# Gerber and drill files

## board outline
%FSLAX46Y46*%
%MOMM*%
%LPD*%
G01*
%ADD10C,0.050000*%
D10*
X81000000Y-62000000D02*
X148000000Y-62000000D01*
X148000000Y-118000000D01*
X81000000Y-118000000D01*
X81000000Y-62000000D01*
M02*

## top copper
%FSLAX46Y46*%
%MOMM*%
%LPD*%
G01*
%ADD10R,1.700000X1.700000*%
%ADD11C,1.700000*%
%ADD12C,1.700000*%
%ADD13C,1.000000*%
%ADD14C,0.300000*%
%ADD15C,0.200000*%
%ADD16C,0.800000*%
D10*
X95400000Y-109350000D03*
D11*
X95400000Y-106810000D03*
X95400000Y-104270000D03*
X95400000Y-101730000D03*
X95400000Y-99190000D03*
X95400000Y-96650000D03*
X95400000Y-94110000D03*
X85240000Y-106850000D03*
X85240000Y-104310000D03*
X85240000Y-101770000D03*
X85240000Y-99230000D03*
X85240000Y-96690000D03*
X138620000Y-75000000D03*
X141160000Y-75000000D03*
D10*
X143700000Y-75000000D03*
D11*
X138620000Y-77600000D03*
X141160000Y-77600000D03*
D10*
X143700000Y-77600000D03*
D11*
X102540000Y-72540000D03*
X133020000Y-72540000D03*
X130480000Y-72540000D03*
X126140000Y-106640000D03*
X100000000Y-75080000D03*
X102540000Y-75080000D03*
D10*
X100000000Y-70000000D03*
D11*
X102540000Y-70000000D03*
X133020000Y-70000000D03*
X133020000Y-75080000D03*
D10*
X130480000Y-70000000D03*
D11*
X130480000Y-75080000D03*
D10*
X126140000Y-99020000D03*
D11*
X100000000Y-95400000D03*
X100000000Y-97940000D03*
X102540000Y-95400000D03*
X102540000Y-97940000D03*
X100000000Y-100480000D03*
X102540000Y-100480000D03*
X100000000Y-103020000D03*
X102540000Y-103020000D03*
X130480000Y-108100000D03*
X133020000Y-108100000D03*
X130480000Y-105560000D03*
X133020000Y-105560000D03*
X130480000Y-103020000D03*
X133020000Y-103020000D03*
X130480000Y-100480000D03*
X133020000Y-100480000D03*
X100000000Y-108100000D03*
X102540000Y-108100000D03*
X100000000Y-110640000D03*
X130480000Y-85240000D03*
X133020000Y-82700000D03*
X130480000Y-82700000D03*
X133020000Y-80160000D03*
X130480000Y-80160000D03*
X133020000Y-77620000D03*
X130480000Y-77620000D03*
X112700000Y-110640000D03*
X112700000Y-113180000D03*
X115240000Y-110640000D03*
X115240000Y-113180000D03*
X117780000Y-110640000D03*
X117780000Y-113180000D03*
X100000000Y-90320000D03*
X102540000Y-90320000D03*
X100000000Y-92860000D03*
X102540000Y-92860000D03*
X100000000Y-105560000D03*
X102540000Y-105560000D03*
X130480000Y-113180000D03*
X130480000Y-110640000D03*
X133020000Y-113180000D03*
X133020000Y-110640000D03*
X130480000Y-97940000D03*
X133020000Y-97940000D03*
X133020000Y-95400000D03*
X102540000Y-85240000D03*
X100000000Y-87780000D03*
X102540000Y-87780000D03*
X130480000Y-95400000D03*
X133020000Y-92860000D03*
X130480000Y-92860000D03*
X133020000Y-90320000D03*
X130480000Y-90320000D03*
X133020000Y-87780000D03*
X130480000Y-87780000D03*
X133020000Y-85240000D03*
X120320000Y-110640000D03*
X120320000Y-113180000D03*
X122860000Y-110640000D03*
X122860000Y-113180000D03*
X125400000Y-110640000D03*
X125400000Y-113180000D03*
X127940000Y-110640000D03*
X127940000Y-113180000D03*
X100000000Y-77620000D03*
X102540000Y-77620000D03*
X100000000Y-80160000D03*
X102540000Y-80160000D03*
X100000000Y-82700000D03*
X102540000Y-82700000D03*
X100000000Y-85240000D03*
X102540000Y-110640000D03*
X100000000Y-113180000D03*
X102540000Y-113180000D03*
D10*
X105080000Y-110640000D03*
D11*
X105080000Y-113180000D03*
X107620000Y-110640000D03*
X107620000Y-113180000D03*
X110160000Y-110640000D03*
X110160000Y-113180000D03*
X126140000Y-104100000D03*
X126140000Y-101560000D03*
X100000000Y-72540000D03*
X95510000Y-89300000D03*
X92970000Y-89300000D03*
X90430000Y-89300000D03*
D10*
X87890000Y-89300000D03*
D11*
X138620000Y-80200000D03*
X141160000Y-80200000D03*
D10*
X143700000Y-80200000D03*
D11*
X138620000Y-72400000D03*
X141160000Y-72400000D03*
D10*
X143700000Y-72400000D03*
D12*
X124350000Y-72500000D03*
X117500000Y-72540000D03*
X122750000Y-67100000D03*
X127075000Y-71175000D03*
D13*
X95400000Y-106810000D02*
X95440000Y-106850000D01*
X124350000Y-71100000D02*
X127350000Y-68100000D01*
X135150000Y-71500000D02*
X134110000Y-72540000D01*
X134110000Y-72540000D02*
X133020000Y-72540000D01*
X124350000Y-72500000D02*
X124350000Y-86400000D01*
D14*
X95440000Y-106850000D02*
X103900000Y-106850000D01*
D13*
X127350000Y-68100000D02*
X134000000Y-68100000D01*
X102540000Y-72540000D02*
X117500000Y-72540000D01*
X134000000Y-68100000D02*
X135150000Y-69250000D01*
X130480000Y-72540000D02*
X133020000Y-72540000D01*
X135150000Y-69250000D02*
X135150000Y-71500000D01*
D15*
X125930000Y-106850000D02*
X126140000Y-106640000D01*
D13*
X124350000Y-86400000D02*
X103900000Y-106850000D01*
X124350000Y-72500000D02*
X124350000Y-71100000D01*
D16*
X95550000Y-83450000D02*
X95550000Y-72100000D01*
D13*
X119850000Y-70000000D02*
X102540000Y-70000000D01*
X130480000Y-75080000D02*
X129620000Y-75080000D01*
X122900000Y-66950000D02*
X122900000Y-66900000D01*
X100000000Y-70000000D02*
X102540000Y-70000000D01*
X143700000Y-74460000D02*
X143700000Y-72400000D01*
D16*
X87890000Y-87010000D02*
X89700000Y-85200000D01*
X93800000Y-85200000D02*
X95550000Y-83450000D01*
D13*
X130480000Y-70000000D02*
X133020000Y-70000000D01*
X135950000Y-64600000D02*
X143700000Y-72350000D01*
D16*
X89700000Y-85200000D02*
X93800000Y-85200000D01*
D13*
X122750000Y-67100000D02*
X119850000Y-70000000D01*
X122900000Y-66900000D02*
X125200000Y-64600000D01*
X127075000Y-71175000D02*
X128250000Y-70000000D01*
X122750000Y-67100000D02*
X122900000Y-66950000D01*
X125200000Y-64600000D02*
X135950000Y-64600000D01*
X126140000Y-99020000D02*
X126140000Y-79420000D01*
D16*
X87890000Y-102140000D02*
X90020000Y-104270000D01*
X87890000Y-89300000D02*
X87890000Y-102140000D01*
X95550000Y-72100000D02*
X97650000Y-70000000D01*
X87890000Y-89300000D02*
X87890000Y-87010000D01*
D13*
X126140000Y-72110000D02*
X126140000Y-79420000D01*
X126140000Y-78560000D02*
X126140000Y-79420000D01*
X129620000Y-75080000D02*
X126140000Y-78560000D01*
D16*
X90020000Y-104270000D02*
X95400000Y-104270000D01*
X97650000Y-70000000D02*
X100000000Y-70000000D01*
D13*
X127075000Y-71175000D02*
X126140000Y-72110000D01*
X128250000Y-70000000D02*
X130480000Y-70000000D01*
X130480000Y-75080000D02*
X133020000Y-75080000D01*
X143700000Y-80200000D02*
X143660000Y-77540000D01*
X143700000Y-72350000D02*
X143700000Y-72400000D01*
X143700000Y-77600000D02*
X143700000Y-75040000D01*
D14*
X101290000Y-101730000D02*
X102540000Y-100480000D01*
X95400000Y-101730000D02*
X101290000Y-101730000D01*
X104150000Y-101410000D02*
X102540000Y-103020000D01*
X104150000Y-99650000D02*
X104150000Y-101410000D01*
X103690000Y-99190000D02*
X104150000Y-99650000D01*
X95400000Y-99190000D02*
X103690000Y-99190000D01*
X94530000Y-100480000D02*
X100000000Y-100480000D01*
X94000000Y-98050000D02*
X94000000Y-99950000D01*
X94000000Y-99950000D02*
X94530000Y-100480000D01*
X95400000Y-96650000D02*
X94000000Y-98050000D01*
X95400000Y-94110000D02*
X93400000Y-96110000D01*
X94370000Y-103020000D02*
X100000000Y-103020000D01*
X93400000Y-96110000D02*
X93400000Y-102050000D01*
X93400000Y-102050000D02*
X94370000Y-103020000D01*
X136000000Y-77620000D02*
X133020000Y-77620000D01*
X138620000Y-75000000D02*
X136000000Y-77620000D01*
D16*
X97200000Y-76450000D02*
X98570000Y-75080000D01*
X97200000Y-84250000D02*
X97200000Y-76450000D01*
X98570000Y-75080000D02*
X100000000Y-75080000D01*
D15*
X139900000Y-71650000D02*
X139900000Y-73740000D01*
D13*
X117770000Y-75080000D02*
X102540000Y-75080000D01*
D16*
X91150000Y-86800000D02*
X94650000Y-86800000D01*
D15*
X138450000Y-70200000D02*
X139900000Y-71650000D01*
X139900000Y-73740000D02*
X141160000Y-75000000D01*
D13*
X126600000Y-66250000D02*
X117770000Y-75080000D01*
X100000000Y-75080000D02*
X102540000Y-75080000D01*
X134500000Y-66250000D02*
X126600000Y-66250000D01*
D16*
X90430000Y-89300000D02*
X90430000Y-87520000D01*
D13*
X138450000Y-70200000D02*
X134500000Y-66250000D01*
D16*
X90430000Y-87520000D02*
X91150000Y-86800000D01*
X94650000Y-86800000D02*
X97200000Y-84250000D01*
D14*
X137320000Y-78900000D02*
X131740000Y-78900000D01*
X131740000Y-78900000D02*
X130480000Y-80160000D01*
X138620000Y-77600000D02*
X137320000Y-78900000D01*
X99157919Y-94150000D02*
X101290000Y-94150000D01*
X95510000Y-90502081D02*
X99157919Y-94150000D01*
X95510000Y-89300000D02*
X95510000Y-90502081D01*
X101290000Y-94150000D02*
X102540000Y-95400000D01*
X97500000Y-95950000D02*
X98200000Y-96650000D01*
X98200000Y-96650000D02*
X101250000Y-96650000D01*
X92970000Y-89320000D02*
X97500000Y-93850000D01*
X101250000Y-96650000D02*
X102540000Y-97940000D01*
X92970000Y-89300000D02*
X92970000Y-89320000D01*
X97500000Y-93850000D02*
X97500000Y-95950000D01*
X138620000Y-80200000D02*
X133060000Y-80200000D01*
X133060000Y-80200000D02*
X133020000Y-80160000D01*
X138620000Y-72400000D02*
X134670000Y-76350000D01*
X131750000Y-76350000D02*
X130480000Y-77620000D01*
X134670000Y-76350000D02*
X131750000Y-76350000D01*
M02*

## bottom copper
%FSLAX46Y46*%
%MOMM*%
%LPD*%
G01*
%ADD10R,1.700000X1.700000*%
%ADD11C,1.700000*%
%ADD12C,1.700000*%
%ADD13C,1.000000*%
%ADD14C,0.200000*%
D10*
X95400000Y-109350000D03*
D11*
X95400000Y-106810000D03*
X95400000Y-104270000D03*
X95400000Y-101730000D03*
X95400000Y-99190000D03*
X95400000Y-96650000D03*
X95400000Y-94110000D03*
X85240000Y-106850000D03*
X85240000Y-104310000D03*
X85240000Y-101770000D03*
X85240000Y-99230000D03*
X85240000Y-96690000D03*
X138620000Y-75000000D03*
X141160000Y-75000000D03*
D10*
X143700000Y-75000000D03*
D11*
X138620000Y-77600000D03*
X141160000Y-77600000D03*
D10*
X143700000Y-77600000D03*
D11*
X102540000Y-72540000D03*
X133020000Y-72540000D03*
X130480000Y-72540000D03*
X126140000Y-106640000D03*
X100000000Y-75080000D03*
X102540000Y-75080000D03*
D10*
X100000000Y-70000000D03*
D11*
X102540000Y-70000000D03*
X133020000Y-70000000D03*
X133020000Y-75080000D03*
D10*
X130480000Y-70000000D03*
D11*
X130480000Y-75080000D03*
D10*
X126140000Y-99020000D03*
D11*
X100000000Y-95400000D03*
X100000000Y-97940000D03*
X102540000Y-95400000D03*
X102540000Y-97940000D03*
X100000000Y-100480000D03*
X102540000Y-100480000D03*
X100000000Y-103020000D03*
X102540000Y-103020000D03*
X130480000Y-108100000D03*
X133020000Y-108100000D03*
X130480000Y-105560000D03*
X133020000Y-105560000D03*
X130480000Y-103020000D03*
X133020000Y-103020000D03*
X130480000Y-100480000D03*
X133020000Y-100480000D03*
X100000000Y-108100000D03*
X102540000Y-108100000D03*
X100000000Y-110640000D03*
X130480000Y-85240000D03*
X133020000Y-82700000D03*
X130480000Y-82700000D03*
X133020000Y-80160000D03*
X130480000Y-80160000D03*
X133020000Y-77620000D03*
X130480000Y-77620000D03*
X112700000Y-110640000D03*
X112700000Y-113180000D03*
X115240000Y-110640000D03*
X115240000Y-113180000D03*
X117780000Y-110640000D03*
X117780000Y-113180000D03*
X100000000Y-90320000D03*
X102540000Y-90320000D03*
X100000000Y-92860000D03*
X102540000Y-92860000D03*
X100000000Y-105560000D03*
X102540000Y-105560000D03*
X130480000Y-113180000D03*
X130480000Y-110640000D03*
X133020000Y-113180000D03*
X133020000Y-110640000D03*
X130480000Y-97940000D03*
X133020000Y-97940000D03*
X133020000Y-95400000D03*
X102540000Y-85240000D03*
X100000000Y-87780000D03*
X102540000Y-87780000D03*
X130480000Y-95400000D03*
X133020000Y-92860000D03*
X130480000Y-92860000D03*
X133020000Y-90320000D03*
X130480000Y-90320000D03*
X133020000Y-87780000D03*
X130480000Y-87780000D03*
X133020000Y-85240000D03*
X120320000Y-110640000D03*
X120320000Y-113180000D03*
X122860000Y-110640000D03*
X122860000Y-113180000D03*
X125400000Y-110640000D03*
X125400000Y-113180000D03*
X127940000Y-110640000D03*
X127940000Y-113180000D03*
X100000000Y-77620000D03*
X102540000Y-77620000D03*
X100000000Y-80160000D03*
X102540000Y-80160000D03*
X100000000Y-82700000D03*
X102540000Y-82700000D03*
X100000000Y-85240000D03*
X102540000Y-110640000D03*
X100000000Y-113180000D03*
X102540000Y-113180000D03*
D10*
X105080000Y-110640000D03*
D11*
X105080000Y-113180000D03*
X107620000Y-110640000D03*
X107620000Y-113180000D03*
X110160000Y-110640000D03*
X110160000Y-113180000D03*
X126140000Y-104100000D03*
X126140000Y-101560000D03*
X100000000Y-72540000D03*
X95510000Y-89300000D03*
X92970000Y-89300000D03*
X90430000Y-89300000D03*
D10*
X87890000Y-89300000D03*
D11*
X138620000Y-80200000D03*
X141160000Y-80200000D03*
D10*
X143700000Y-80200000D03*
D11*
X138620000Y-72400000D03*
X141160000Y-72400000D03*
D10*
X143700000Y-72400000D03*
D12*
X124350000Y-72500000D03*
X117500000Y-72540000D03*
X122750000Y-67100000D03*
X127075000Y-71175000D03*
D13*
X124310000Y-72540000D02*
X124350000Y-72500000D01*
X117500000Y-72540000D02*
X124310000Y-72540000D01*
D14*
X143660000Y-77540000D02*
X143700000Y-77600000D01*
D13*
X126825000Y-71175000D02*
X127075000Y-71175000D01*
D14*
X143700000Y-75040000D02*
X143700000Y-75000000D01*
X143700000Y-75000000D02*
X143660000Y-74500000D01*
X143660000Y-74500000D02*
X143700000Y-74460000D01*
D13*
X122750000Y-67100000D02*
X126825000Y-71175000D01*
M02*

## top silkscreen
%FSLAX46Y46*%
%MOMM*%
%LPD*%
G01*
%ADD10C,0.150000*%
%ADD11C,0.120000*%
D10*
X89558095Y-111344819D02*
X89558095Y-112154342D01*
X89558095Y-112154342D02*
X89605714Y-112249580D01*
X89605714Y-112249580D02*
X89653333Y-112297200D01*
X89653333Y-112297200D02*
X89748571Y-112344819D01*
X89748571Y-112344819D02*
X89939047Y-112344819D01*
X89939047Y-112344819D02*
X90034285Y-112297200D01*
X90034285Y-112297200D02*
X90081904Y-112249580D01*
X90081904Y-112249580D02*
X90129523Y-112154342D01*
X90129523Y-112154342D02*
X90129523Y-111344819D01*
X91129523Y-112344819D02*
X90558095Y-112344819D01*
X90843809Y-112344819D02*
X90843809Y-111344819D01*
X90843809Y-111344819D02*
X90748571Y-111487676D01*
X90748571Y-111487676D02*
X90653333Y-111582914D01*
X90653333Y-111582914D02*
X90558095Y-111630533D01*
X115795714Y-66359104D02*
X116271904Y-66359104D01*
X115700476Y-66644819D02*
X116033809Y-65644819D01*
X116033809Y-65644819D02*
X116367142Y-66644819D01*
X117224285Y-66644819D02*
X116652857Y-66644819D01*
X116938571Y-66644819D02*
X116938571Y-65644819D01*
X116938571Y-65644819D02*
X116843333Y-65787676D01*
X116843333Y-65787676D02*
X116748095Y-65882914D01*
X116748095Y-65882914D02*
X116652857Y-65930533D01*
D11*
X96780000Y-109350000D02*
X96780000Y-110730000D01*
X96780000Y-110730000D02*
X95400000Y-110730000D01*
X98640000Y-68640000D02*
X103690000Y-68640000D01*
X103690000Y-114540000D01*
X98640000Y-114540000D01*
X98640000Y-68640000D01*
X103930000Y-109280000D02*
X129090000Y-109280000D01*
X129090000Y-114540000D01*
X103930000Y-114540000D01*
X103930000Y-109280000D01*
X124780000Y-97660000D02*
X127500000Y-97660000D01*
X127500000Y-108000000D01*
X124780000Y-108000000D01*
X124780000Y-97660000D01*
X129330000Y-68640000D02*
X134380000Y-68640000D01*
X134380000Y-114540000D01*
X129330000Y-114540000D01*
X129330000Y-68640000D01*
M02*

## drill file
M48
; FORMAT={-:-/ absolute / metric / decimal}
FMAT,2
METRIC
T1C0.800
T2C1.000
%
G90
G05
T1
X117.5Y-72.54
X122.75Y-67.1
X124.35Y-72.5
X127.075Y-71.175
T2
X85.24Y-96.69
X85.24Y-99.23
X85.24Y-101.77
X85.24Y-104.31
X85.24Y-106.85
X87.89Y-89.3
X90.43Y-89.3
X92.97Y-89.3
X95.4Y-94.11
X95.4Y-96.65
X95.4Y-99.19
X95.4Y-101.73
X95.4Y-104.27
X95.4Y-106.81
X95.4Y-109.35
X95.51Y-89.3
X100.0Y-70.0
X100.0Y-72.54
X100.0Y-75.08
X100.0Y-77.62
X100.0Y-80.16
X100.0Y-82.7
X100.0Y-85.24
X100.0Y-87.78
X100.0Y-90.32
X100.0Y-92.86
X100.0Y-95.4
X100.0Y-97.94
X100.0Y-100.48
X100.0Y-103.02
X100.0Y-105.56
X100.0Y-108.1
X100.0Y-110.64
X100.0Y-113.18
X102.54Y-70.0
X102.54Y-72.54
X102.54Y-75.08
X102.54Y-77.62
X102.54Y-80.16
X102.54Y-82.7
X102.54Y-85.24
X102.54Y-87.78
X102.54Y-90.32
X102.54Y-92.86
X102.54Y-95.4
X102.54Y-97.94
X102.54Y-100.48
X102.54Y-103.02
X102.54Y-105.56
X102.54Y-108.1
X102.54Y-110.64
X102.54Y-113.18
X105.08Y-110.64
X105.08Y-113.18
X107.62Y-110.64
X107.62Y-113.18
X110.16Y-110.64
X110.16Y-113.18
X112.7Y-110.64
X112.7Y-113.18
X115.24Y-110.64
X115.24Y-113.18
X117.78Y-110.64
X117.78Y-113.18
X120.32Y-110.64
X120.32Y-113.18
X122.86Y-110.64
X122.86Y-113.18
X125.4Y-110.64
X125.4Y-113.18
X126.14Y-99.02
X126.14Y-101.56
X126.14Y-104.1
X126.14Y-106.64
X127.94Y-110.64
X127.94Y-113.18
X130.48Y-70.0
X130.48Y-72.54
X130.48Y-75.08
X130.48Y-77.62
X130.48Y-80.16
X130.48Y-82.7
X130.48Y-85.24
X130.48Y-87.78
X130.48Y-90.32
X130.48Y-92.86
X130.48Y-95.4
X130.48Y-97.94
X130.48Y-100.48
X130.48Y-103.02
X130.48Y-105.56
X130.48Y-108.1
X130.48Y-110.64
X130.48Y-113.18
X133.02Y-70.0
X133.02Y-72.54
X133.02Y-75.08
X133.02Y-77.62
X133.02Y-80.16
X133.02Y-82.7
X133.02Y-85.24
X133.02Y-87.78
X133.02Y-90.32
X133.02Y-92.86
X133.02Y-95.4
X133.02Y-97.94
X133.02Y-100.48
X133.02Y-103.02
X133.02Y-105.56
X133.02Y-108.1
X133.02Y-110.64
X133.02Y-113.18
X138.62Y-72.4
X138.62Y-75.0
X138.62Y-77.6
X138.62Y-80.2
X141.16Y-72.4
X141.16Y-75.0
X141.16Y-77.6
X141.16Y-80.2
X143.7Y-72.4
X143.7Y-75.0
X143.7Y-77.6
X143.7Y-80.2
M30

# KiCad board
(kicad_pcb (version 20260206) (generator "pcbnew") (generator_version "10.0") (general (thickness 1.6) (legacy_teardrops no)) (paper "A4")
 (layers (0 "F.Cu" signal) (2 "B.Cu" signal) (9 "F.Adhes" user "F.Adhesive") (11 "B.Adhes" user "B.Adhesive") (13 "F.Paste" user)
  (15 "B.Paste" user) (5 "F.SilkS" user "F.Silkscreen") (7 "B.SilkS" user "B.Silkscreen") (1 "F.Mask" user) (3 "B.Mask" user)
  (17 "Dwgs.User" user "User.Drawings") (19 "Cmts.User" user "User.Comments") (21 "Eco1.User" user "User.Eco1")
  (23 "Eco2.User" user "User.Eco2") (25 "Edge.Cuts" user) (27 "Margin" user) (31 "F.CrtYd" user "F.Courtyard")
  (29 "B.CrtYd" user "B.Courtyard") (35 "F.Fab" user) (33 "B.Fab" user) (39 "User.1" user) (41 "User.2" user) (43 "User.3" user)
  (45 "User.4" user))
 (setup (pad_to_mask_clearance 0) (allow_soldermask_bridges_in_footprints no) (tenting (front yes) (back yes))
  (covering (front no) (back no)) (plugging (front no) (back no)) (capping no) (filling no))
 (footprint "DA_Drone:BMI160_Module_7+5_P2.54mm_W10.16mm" (layer "F.Cu") (at 95.4 109.35 180)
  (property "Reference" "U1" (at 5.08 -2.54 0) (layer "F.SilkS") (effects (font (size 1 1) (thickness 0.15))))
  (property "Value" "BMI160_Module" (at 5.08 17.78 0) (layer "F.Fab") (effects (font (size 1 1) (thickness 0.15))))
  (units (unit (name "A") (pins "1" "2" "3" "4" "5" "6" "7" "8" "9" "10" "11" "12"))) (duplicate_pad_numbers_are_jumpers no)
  (fp_line (start -1.38 0) (end -1.38 -1.38) (stroke (width 0.12) (type default)) (layer "F.SilkS"))
  (fp_line (start -1.38 -1.38) (end 0 -1.38) (stroke (width 0.12) (type default)) (layer "F.SilkS"))
  (pad "1" thru_hole rect (at 0 0 180) (size 1.7 1.7) (drill 1) (layers "*.Cu" "*.Mask") (remove_unused_layers no)
   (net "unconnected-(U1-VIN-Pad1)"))
  (pad "2" thru_hole circle (at 0 2.54 180) (size 1.7 1.7) (drill 1) (layers "*.Cu" "*.Mask") (remove_unused_layers no) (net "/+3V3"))
  (pad "3" thru_hole circle (at 0 5.08 180) (size 1.7 1.7) (drill 1) (layers "*.Cu" "*.Mask") (remove_unused_layers no) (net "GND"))
  (pad "4" thru_hole circle (at 0 7.62 180) (size 1.7 1.7) (drill 1) (layers "*.Cu" "*.Mask") (remove_unused_layers no) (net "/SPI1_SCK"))
  (pad "5" thru_hole circle (at 0 10.16 180) (size 1.7 1.7) (drill 1) (layers "*.Cu" "*.Mask") (remove_unused_layers no) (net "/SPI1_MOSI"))
  (pad "6" thru_hole circle (at 0 12.7 180) (size 1.7 1.7) (drill 1) (layers "*.Cu" "*.Mask") (remove_unused_layers no) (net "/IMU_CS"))
  (pad "7" thru_hole circle (at 0 15.24 180) (size 1.7 1.7) (drill 1) (layers "*.Cu" "*.Mask") (remove_unused_layers no) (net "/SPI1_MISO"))
  (pad "8" thru_hole circle (at 10.16 2.5 180) (size 1.7 1.7) (drill 1) (layers "*.Cu" "*.Mask") (remove_unused_layers no)
   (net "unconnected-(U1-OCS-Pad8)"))
  (pad "9" thru_hole circle (at 10.16 5.04 180) (size 1.7 1.7) (drill 1) (layers "*.Cu" "*.Mask") (remove_unused_layers no)
   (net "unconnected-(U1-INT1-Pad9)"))
  (pad "10" thru_hole circle (at 10.16 7.58 180) (size 1.7 1.7) (drill 1) (layers "*.Cu" "*.Mask") (remove_unused_layers no)
   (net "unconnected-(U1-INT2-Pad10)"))
  (pad "11" thru_hole circle (at 10.16 10.12 180) (size 1.7 1.7) (drill 1) (layers "*.Cu" "*.Mask") (remove_unused_layers no)
   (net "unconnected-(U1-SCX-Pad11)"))
  (pad "12" thru_hole circle (at 10.16 12.66 180) (size 1.7 1.7) (drill 1) (layers "*.Cu" "*.Mask") (remove_unused_layers no)
   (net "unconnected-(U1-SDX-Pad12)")))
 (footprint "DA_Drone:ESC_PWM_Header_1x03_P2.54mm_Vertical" (layer "F.Cu") (at 143.7 75 -90)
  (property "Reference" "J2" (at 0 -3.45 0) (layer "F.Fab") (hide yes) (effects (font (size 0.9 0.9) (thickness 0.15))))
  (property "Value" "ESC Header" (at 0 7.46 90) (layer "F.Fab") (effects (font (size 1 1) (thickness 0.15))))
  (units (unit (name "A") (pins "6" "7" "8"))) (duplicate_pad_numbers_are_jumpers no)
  (pad "6" thru_hole circle (at 0 5.08 270) (size 1.7 1.7) (drill 1) (layers "*.Cu" "*.Mask") (remove_unused_layers no) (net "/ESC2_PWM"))
  (pad "7" thru_hole circle (at 0 2.54 270) (size 1.7 1.7) (drill 1) (layers "*.Cu" "*.Mask") (remove_unused_layers no) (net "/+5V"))
  (pad "8" thru_hole rect (at 0 0 270) (size 1.7 1.7) (drill 1) (layers "*.Cu" "*.Mask") (remove_unused_layers no) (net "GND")))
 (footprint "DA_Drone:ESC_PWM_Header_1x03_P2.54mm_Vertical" (layer "F.Cu") (at 143.7 77.6 -90)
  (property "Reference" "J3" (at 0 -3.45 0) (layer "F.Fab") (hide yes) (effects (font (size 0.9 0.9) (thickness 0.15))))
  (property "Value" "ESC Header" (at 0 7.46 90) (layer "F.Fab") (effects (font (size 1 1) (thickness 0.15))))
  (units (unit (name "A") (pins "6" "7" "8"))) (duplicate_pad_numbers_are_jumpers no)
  (pad "6" thru_hole circle (at 0 5.08 270) (size 1.7 1.7) (drill 1) (layers "*.Cu" "*.Mask") (remove_unused_layers no) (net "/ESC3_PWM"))
  (pad "7" thru_hole circle (at 0 2.54 270) (size 1.7 1.7) (drill 1) (layers "*.Cu" "*.Mask") (remove_unused_layers no)
   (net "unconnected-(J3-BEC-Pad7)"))
  (pad "8" thru_hole rect (at 0 0 270) (size 1.7 1.7) (drill 1) (layers "*.Cu" "*.Mask") (remove_unused_layers no) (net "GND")))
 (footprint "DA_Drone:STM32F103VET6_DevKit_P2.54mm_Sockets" (layer "F.Cu") (at 100 70)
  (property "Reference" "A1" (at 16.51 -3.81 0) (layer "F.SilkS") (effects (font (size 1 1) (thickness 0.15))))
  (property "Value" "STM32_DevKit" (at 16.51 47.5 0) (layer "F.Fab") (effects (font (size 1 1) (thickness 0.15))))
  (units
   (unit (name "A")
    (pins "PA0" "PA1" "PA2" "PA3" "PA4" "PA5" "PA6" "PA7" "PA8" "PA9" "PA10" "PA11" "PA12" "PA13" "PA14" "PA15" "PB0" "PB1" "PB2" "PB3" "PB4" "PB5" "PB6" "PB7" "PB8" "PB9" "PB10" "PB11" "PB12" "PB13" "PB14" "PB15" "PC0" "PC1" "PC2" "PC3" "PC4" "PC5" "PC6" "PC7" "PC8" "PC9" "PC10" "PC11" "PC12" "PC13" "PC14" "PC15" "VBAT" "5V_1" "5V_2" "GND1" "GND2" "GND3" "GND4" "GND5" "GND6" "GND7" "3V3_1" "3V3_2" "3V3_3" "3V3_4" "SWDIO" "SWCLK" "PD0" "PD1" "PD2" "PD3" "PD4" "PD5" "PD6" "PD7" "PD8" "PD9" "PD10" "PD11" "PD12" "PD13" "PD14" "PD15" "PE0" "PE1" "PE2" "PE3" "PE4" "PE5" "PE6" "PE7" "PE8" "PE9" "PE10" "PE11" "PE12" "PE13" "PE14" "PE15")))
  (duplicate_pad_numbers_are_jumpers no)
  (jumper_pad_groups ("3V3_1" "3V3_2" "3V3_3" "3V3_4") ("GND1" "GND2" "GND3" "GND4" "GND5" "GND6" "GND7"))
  (fp_rect (start -1.36 -1.36) (end 3.69 44.54) (stroke (width 0.12) (type solid)) (fill no) (layer "F.SilkS"))
  (fp_rect (start 3.93 39.28) (end 29.09 44.54) (stroke (width 0.12) (type solid)) (fill no) (layer "F.SilkS"))
  (fp_rect (start 24.78 27.66) (end 27.5 38) (stroke (width 0.12) (type solid)) (fill no) (layer "F.SilkS"))
  (fp_rect (start 29.33 -1.36) (end 34.38 44.54) (stroke (width 0.12) (type solid)) (fill no) (layer "F.SilkS"))
  (pad "3V3_1" thru_hole circle (at 2.54 2.54) (size 1.7 1.7) (drill 1) (layers "*.Cu" "*.Mask") (remove_unused_layers no) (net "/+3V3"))
  (pad "3V3_2" thru_hole circle (at 33.02 2.54) (size 1.7 1.7) (drill 1) (layers "*.Cu" "*.Mask") (remove_unused_layers no) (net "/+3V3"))
  (pad "3V3_3" thru_hole circle (at 30.48 2.54) (size 1.7 1.7) (drill 1) (layers "*.Cu" "*.Mask") (remove_unused_layers no) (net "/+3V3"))
  (pad "3V3_4" thru_hole circle (at 26.14 36.64) (size 1.7 1.7) (drill 1) (layers "*.Cu" "*.Mask") (remove_unused_layers no) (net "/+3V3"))
  (pad "5V_1" thru_hole circle (at 0 5.08) (size 1.7 1.7) (drill 1) (layers "*.Cu" "*.Mask") (remove_unused_layers no) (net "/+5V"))
  (pad "5V_2" thru_hole circle (at 2.54 5.08) (size 1.7 1.7) (drill 1) (layers "*.Cu" "*.Mask") (remove_unused_layers no) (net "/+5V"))
  (pad "GND1" thru_hole rect (at 0 0) (size 1.7 1.7) (drill 1) (layers "*.Cu" "*.Mask") (remove_unused_layers no) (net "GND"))
  (pad "GND2" thru_hole circle (at 2.54 0) (size 1.7 1.7) (drill 1) (layers "*.Cu" "*.Mask") (remove_unused_layers no) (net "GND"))
  (pad "GND3" thru_hole circle (at 33.02 0) (size 1.7 1.7) (drill 1) (layers "*.Cu" "*.Mask") (remove_unused_layers no) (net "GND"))
  (pad "GND4" thru_hole circle (at 33.02 5.08) (size 1.7 1.7) (drill 1) (layers "*.Cu" "*.Mask") (remove_unused_layers no) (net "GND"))
  (pad "GND5" thru_hole rect (at 30.48 0) (size 1.7 1.7) (drill 1) (layers "*.Cu" "*.Mask") (remove_unused_layers no) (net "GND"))
  (pad "GND6" thru_hole circle (at 30.48 5.08) (size 1.7 1.7) (drill 1) (layers "*.Cu" "*.Mask") (remove_unused_layers no) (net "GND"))
  (pad "GND7" thru_hole rect (at 26.14 29.02) (size 1.7 1.7) (drill 1) (layers "*.Cu" "*.Mask") (remove_unused_layers no) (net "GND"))
  (pad "PA0" thru_hole circle (at 0 25.4) (size 1.7 1.7) (drill 1) (layers "*.Cu" "*.Mask") (remove_unused_layers no)
   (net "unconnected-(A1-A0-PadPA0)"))
  (pad "PA1" thru_hole circle (at 0 27.94) (size 1.7 1.7) (drill 1) (layers "*.Cu" "*.Mask") (remove_unused_layers no)
   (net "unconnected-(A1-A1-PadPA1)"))
  (pad "PA2" thru_hole circle (at 2.54 25.4) (size 1.7 1.7) (drill 1) (layers "*.Cu" "*.Mask") (remove_unused_layers no)
   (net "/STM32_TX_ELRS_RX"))
  (pad "PA3" thru_hole circle (at 2.54 27.94) (size 1.7 1.7) (drill 1) (layers "*.Cu" "*.Mask") (remove_unused_layers no)
   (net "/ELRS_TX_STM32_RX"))
  (pad "PA4" thru_hole circle (at 0 30.48) (size 1.7 1.7) (drill 1) (layers "*.Cu" "*.Mask") (remove_unused_layers no) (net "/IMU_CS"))
  (pad "PA5" thru_hole circle (at 2.54 30.48) (size 1.7 1.7) (drill 1) (layers "*.Cu" "*.Mask") (remove_unused_layers no) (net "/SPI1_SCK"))
  (pad "PA6" thru_hole circle (at 0 33.02) (size 1.7 1.7) (drill 1) (layers "*.Cu" "*.Mask") (remove_unused_layers no) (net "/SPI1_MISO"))
  (pad "PA7" thru_hole circle (at 2.54 33.02) (size 1.7 1.7) (drill 1) (layers "*.Cu" "*.Mask") (remove_unused_layers no) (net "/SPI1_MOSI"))
  (pad "PA8" thru_hole circle (at 30.48 38.1) (size 1.7 1.7) (drill 1) (layers "*.Cu" "*.Mask") (remove_unused_layers no)
   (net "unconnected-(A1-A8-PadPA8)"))
  (pad "PA9" thru_hole circle (at 33.02 38.1) (size 1.7 1.7) (drill 1) (layers "*.Cu" "*.Mask") (remove_unused_layers no)
   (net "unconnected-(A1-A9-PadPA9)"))
  (pad "PA10" thru_hole circle (at 30.48 35.56) (size 1.7 1.7) (drill 1) (layers "*.Cu" "*.Mask") (remove_unused_layers no)
   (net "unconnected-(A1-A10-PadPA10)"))
  (pad "PA11" thru_hole circle (at 33.02 35.56) (size 1.7 1.7) (drill 1) (layers "*.Cu" "*.Mask") (remove_unused_layers no)
   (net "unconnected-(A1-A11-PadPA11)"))
  (pad "PA12" thru_hole circle (at 30.48 33.02) (size 1.7 1.7) (drill 1) (layers "*.Cu" "*.Mask") (remove_unused_layers no)
   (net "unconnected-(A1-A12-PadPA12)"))
  (pad "PA13" thru_hole circle (at 33.02 33.02) (size 1.7 1.7) (drill 1) (layers "*.Cu" "*.Mask") (remove_unused_layers no)
   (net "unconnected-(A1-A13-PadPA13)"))
  (pad "PA14" thru_hole circle (at 30.48 30.48) (size 1.7 1.7) (drill 1) (layers "*.Cu" "*.Mask") (remove_unused_layers no)
   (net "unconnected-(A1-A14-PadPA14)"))
  (pad "PA15" thru_hole circle (at 33.02 30.48) (size 1.7 1.7) (drill 1) (layers "*.Cu" "*.Mask") (remove_unused_layers no)
   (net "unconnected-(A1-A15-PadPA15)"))
  (pad "PB0" thru_hole circle (at 0 38.1) (size 1.7 1.7) (drill 1) (layers "*.Cu" "*.Mask") (remove_unused_layers no)
   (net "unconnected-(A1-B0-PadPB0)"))
  (pad "PB1" thru_hole circle (at 2.54 38.1) (size 1.7 1.7) (drill 1) (layers "*.Cu" "*.Mask") (remove_unused_layers no)
   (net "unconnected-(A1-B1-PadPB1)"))
  (pad "PB2" thru_hole circle (at 0 40.64) (size 1.7 1.7) (drill 1) (layers "*.Cu" "*.Mask") (remove_unused_layers no)
   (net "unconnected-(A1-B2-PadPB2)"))
  (pad "PB3" thru_hole circle (at 30.48 15.24) (size 1.7 1.7) (drill 1) (layers "*.Cu" "*.Mask") (remove_unused_layers no)
   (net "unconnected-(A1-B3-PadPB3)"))
  (pad "PB4" thru_hole circle (at 33.02 12.7) (size 1.7 1.7) (drill 1) (layers "*.Cu" "*.Mask") (remove_unused_layers no)
   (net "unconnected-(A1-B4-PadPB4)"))
  (pad "PB5" thru_hole circle (at 30.48 12.7) (size 1.7 1.7) (drill 1) (layers "*.Cu" "*.Mask") (remove_unused_layers no)
   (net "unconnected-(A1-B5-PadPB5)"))
  (pad "PB6" thru_hole circle (at 33.02 10.16) (size 1.7 1.7) (drill 1) (layers "*.Cu" "*.Mask") (remove_unused_layers no) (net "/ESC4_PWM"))
  (pad "PB7" thru_hole circle (at 30.48 10.16) (size 1.7 1.7) (drill 1) (layers "*.Cu" "*.Mask") (remove_unused_layers no) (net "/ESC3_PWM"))
  (pad "PB8" thru_hole circle (at 33.02 7.62) (size 1.7 1.7) (drill 1) (layers "*.Cu" "*.Mask") (remove_unused_layers no) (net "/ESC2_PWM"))
  (pad "PB9" thru_hole circle (at 30.48 7.62) (size 1.7 1.7) (drill 1) (layers "*.Cu" "*.Mask") (remove_unused_layers no) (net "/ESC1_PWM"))
  (pad "PB10" thru_hole circle (at 12.7 40.64) (size 1.7 1.7) (drill 1) (layers "*.Cu" "*.Mask") (remove_unused_layers no)
   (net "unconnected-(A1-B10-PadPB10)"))
  (pad "PB11" thru_hole circle (at 12.7 43.18) (size 1.7 1.7) (drill 1) (layers "*.Cu" "*.Mask") (remove_unused_layers no)
   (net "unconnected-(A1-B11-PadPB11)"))
  (pad "PB12" thru_hole circle (at 15.24 40.64) (size 1.7 1.7) (drill 1) (layers "*.Cu" "*.Mask") (remove_unused_layers no)
   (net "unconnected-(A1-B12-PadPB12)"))
  (pad "PB13" thru_hole circle (at 15.24 43.18) (size 1.7 1.7) (drill 1) (layers "*.Cu" "*.Mask") (remove_unused_layers no)
   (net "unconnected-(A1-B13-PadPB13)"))
  (pad "PB14" thru_hole circle (at 17.78 40.64) (size 1.7 1.7) (drill 1) (layers "*.Cu" "*.Mask") (remove_unused_layers no)
   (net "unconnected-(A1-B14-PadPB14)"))
  (pad "PB15" thru_hole circle (at 17.78 43.18) (size 1.7 1.7) (drill 1) (layers "*.Cu" "*.Mask") (remove_unused_layers no)
   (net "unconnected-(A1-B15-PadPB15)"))
  (pad "PC0" thru_hole circle (at 0 20.32) (size 1.7 1.7) (drill 1) (layers "*.Cu" "*.Mask") (remove_unused_layers no)
   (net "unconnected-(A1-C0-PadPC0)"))
  (pad "PC1" thru_hole circle (at 2.54 20.32) (size 1.7 1.7) (drill 1) (layers "*.Cu" "*.Mask") (remove_unused_layers no)
   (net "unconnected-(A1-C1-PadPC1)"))
  (pad "PC2" thru_hole circle (at 0 22.86) (size 1.7 1.7) (drill 1) (layers "*.Cu" "*.Mask") (remove_unused_layers no)
   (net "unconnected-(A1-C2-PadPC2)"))
  (pad "PC3" thru_hole circle (at 2.54 22.86) (size 1.7 1.7) (drill 1) (layers "*.Cu" "*.Mask") (remove_unused_layers no)
   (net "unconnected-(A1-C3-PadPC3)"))
  (pad "PC4" thru_hole circle (at 0 35.56) (size 1.7 1.7) (drill 1) (layers "*.Cu" "*.Mask") (remove_unused_layers no)
   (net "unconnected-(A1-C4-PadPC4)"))
  (pad "PC5" thru_hole circle (at 2.54 35.56) (size 1.7 1.7) (drill 1) (layers "*.Cu" "*.Mask") (remove_unused_layers no)
   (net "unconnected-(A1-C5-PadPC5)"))
  (pad "PC6" thru_hole circle (at 30.48 43.18) (size 1.7 1.7) (drill 1) (layers "*.Cu" "*.Mask") (remove_unused_layers no)
   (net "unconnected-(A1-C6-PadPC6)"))
  (pad "PC7" thru_hole circle (at 30.48 40.64) (size 1.7 1.7) (drill 1) (layers "*.Cu" "*.Mask") (remove_unused_layers no)
   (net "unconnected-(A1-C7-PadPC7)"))
  (pad "PC8" thru_hole circle (at 33.02 43.18) (size 1.7 1.7) (drill 1) (layers "*.Cu" "*.Mask") (remove_unused_layers no)
   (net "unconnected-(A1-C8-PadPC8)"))
  (pad "PC9" thru_hole circle (at 33.02 40.64) (size 1.7 1.7) (drill 1) (layers "*.Cu" "*.Mask") (remove_unused_layers no)
   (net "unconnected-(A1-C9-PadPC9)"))
  (pad "PC10" thru_hole circle (at 30.48 27.94) (size 1.7 1.7) (drill 1) (layers "*.Cu" "*.Mask") (remove_unused_layers no)
   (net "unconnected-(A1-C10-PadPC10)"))
  (pad "PC11" thru_hole circle (at 33.02 27.94) (size 1.7 1.7) (drill 1) (layers "*.Cu" "*.Mask") (remove_unused_layers no)
   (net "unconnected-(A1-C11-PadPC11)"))
  (pad "PC12" thru_hole circle (at 33.02 25.4) (size 1.7 1.7) (drill 1) (layers "*.Cu" "*.Mask") (remove_unused_layers no)
   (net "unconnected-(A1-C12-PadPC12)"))
  (pad "PC13" thru_hole circle (at 2.54 15.24) (size 1.7 1.7) (drill 1) (layers "*.Cu" "*.Mask") (remove_unused_layers no)
   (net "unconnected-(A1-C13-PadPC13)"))
  (pad "PC14" thru_hole circle (at 0 17.78) (size 1.7 1.7) (drill 1) (layers "*.Cu" "*.Mask") (remove_unused_layers no)
   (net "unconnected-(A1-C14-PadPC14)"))
  (pad "PC15" thru_hole circle (at 2.54 17.78) (size 1.7 1.7) (drill 1) (layers "*.Cu" "*.Mask") (remove_unused_layers no)
   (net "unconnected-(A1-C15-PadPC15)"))
  (pad "PD0" thru_hole circle (at 30.48 25.4) (size 1.7 1.7) (drill 1) (layers "*.Cu" "*.Mask") (remove_unused_layers no)
   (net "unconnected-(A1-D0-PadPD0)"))
  (pad "PD1" thru_hole circle (at 33.02 22.86) (size 1.7 1.7) (drill 1) (layers "*.Cu" "*.Mask") (remove_unused_layers no)
   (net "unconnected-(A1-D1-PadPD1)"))
  (pad "PD2" thru_hole circle (at 30.48 22.86) (size 1.7 1.7) (drill 1) (layers "*.Cu" "*.Mask") (remove_unused_layers no)
   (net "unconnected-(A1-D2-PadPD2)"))
  (pad "PD3" thru_hole circle (at 33.02 20.32) (size 1.7 1.7) (drill 1) (layers "*.Cu" "*.Mask") (remove_unused_layers no)
   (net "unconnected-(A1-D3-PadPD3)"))
  (pad "PD4" thru_hole circle (at 30.48 20.32) (size 1.7 1.7) (drill 1) (layers "*.Cu" "*.Mask") (remove_unused_layers no)
   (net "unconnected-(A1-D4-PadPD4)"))
  (pad "PD5" thru_hole circle (at 33.02 17.78) (size 1.7 1.7) (drill 1) (layers "*.Cu" "*.Mask") (remove_unused_layers no)
   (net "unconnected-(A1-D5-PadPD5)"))
  (pad "PD6" thru_hole circle (at 30.48 17.78) (size 1.7 1.7) (drill 1) (layers "*.Cu" "*.Mask") (remove_unused_layers no)
   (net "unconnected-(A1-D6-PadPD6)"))
  (pad "PD7" thru_hole circle (at 33.02 15.24) (size 1.7 1.7) (drill 1) (layers "*.Cu" "*.Mask") (remove_unused_layers no)
   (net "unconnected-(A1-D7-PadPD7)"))
  (pad "PD8" thru_hole circle (at 20.32 40.64) (size 1.7 1.7) (drill 1) (layers "*.Cu" "*.Mask") (remove_unused_layers no)
   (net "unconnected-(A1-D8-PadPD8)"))
  (pad "PD9" thru_hole circle (at 20.32 43.18) (size 1.7 1.7) (drill 1) (layers "*.Cu" "*.Mask") (remove_unused_layers no)
   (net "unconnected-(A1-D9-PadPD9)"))
  (pad "PD10" thru_hole circle (at 22.86 40.64) (size 1.7 1.7) (drill 1) (layers "*.Cu" "*.Mask") (remove_unused_layers no)
   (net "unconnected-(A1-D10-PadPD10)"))
  (pad "PD11" thru_hole circle (at 22.86 43.18) (size 1.7 1.7) (drill 1) (layers "*.Cu" "*.Mask") (remove_unused_layers no)
   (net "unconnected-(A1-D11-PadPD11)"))
  (pad "PD12" thru_hole circle (at 25.4 40.64) (size 1.7 1.7) (drill 1) (layers "*.Cu" "*.Mask") (remove_unused_layers no)
   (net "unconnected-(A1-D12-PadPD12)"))
  (pad "PD13" thru_hole circle (at 25.4 43.18) (size 1.7 1.7) (drill 1) (layers "*.Cu" "*.Mask") (remove_unused_layers no)
   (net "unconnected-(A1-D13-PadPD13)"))
  (pad "PD14" thru_hole circle (at 27.94 40.64) (size 1.7 1.7) (drill 1) (layers "*.Cu" "*.Mask") (remove_unused_layers no)
   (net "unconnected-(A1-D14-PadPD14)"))
  (pad "PD15" thru_hole circle (at 27.94 43.18) (size 1.7 1.7) (drill 1) (layers "*.Cu" "*.Mask") (remove_unused_layers no)
   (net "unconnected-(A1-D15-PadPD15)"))
  (pad "PE0" thru_hole circle (at 0 7.62) (size 1.7 1.7) (drill 1) (layers "*.Cu" "*.Mask") (remove_unused_layers no)
   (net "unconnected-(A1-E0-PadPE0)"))
  (pad "PE1" thru_hole circle (at 2.54 7.62) (size 1.7 1.7) (drill 1) (layers "*.Cu" "*.Mask") (remove_unused_layers no)
   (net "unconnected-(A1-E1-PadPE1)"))
  (pad "PE2" thru_hole circle (at 0 10.16) (size 1.7 1.7) (drill 1) (layers "*.Cu" "*.Mask") (remove_unused_layers no)
   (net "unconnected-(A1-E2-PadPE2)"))
  (pad "PE3" thru_hole circle (at 2.54 10.16) (size 1.7 1.7) (drill 1) (layers "*.Cu" "*.Mask") (remove_unused_layers no)
   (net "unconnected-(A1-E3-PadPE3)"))
  (pad "PE4" thru_hole circle (at 0 12.7) (size 1.7 1.7) (drill 1) (layers "*.Cu" "*.Mask") (remove_unused_layers no)
   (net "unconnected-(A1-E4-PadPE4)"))
  (pad "PE5" thru_hole circle (at 2.54 12.7) (size 1.7 1.7) (drill 1) (layers "*.Cu" "*.Mask") (remove_unused_layers no)
   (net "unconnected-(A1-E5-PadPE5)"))
  (pad "PE6" thru_hole circle (at 0 15.24) (size 1.7 1.7) (drill 1) (layers "*.Cu" "*.Mask") (remove_unused_layers no)
   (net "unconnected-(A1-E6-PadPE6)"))
  (pad "PE7" thru_hole circle (at 2.54 40.64) (size 1.7 1.7) (drill 1) (layers "*.Cu" "*.Mask") (remove_unused_layers no)
   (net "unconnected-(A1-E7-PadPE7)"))
  (pad "PE8" thru_hole circle (at 0 43.18) (size 1.7 1.7) (drill 1) (layers "*.Cu" "*.Mask") (remove_unused_layers no)
   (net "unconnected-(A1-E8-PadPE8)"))
  (pad "PE9" thru_hole circle (at 2.54 43.18) (size 1.7 1.7) (drill 1) (layers "*.Cu" "*.Mask") (remove_unused_layers no)
   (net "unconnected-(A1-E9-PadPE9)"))
  (pad "PE10" thru_hole rect (at 5.08 40.64) (size 1.7 1.7) (drill 1) (layers "*.Cu" "*.Mask") (remove_unused_layers no)
   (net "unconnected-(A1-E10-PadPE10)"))
  (pad "PE11" thru_hole circle (at 5.08 43.18) (size 1.7 1.7) (drill 1) (layers "*.Cu" "*.Mask") (remove_unused_layers no)
   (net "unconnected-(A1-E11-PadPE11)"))
  (pad "PE12" thru_hole circle (at 7.62 40.64) (size 1.7 1.7) (drill 1) (layers "*.Cu" "*.Mask") (remove_unused_layers no)
   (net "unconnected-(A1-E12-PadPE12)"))
  (pad "PE13" thru_hole circle (at 7.62 43.18) (size 1.7 1.7) (drill 1) (layers "*.Cu" "*.Mask") (remove_unused_layers no)
   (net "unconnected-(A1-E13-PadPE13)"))
  (pad "PE14" thru_hole circle (at 10.16 40.64) (size 1.7 1.7) (drill 1) (layers "*.Cu" "*.Mask") (remove_unused_layers no)
   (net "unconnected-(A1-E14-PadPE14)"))
  (pad "PE15" thru_hole circle (at 10.16 43.18) (size 1.7 1.7) (drill 1) (layers "*.Cu" "*.Mask") (remove_unused_layers no)
   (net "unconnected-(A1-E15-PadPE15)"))
  (pad "SWCLK" thru_hole circle (at 26.14 34.1) (size 1.7 1.7) (drill 1) (layers "*.Cu" "*.Mask") (remove_unused_layers no)
   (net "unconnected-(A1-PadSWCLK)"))
  (pad "SWDIO" thru_hole circle (at 26.14 31.56) (size 1.7 1.7) (drill 1) (layers "*.Cu" "*.Mask") (remove_unused_layers no)
   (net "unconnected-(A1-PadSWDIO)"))
  (pad "VBAT" thru_hole circle (at 0 2.54) (size 1.7 1.7) (drill 1) (layers "*.Cu" "*.Mask") (remove_unused_layers no)
   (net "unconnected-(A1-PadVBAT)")))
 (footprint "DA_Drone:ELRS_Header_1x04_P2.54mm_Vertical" (layer "F.Cu") (at 87.89 89.3 90)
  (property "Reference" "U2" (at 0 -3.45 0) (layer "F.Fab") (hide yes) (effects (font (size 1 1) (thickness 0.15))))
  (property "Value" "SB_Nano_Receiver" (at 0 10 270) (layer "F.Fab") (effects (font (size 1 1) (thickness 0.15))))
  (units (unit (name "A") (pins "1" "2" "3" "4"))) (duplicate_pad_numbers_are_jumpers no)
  (pad "1" thru_hole circle (at 0 7.62 90) (size 1.7 1.7) (drill 1) (layers "*.Cu" "*.Mask") (remove_unused_layers no)
   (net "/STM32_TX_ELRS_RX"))
  (pad "2" thru_hole circle (at 0 5.08 90) (size 1.7 1.7) (drill 1) (layers "*.Cu" "*.Mask") (remove_unused_layers no)
   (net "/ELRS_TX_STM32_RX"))
  (pad "3" thru_hole circle (at 0 2.54 90) (size 1.7 1.7) (drill 1) (layers "*.Cu" "*.Mask") (remove_unused_layers no) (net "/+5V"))
  (pad "4" thru_hole rect (at 0 0 90) (size 1.7 1.7) (drill 1) (layers "*.Cu" "*.Mask") (remove_unused_layers no) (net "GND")))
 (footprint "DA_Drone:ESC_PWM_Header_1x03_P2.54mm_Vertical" (layer "F.Cu") (at 143.7 80.2 -90)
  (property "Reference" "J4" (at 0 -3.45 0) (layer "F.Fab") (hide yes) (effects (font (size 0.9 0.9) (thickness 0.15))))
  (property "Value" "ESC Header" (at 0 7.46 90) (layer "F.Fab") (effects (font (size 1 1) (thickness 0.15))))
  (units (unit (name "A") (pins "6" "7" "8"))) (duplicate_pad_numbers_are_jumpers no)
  (pad "6" thru_hole circle (at 0 5.08 270) (size 1.7 1.7) (drill 1) (layers "*.Cu" "*.Mask") (remove_unused_layers no) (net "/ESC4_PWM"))
  (pad "7" thru_hole circle (at 0 2.54 270) (size 1.7 1.7) (drill 1) (layers "*.Cu" "*.Mask") (remove_unused_layers no)
   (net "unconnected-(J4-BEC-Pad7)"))
  (pad "8" thru_hole rect (at 0 0 270) (size 1.7 1.7) (drill 1) (layers "*.Cu" "*.Mask") (remove_unused_layers no) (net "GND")))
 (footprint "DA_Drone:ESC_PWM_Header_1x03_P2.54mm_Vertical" (layer "F.Cu") (at 143.7 72.4 -90)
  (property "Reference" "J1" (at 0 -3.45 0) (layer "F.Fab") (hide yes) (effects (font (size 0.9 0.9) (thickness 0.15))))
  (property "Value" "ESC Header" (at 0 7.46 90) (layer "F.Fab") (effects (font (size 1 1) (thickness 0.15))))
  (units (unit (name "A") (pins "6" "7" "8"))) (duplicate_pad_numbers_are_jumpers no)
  (pad "6" thru_hole circle (at 0 5.08 270) (size 1.7 1.7) (drill 1) (layers "*.Cu" "*.Mask") (remove_unused_layers no) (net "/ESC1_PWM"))
  (pad "7" thru_hole circle (at 0 2.54 270) (size 1.7 1.7) (drill 1) (layers "*.Cu" "*.Mask") (remove_unused_layers no)
   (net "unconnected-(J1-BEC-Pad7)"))
  (pad "8" thru_hole rect (at 0 0 270) (size 1.7 1.7) (drill 1) (layers "*.Cu" "*.Mask") (remove_unused_layers no) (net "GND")))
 (gr_rect (start 81 62) (end 148 118) (stroke (width 0.05) (type default)) (fill no) (layer "Edge.Cuts"))
 (segment (start 95.4 106.81) (end 95.44 106.85) (width 1) (layer "F.Cu") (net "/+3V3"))
 (segment (start 124.35 71.1) (end 127.35 68.1) (width 1) (layer "F.Cu") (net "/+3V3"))
 (segment (start 135.15 71.5) (end 134.11 72.54) (width 1) (layer "F.Cu") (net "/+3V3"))
 (segment (start 134.11 72.54) (end 133.02 72.54) (width 1) (layer "F.Cu") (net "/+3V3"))
 (segment (start 124.35 72.5) (end 124.35 86.4) (width 1) (layer "F.Cu") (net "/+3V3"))
 (segment (start 95.44 106.85) (end 103.9 106.85) (width 0.3) (layer "F.Cu") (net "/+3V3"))
 (segment (start 127.35 68.1) (end 134 68.1) (width 1) (layer "F.Cu") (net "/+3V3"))
 (segment (start 102.54 72.54) (end 117.5 72.54) (width 1) (layer "F.Cu") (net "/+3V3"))
 (segment (start 134 68.1) (end 135.15 69.25) (width 1) (layer "F.Cu") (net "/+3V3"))
 (segment (start 130.48 72.54) (end 133.02 72.54) (width 1) (layer "F.Cu") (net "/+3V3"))
 (segment (start 135.15 69.25) (end 135.15 71.5) (width 1) (layer "F.Cu") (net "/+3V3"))
 (segment (start 125.93 106.85) (end 126.14 106.64) (width 0.2) (layer "F.Cu") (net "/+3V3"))
 (segment (start 124.35 86.4) (end 103.9 106.85) (width 1) (layer "F.Cu") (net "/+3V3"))
 (segment (start 124.35 72.5) (end 124.35 71.1) (width 1) (layer "F.Cu") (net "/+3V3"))
 (via (at 124.35 72.5) (size 1.7) (drill 0.8) (layers "F.Cu" "B.Cu") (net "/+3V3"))
 (via (at 117.5 72.54) (size 1.7) (drill 0.8) (layers "F.Cu" "B.Cu") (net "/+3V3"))
 (segment (start 124.31 72.54) (end 124.35 72.5) (width 1) (layer "B.Cu") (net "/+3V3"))
 (segment (start 117.5 72.54) (end 124.31 72.54) (width 1) (layer "B.Cu") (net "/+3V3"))
 (segment (start 95.55 83.45) (end 95.55 72.1) (width 0.8) (layer "F.Cu") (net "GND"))
 (segment (start 119.85 70) (end 102.54 70) (width 1) (layer "F.Cu") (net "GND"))
 (segment (start 130.48 75.08) (end 129.62 75.08) (width 1) (layer "F.Cu") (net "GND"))
 (segment (start 122.9 66.95) (end 122.9 66.9) (width 1) (layer "F.Cu") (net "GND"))
 (segment (start 100 70) (end 102.54 70) (width 1) (layer "F.Cu") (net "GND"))
 (segment (start 143.7 74.46) (end 143.7 72.4) (width 1) (layer "F.Cu") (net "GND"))
 (segment (start 87.89 87.01) (end 89.7 85.2) (width 0.8) (layer "F.Cu") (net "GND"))
 (segment (start 93.8 85.2) (end 95.55 83.45) (width 0.8) (layer "F.Cu") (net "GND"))
 (segment (start 130.48 70) (end 133.02 70) (width 1) (layer "F.Cu") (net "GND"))
 (segment (start 135.95 64.6) (end 143.7 72.35) (width 1) (layer "F.Cu") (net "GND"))
 (segment (start 89.7 85.2) (end 93.8 85.2) (width 0.8) (layer "F.Cu") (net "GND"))
 (segment (start 122.75 67.1) (end 119.85 70) (width 1) (layer "F.Cu") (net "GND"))
 (segment (start 122.9 66.9) (end 125.2 64.6) (width 1) (layer "F.Cu") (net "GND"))
 (segment (start 127.075 71.175) (end 128.25 70) (width 1) (layer "F.Cu") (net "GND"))
 (segment (start 122.75 67.1) (end 122.9 66.95) (width 1) (layer "F.Cu") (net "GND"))
 (segment (start 125.2 64.6) (end 135.95 64.6) (width 1) (layer "F.Cu") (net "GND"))
 (segment (start 126.14 99.02) (end 126.14 79.42) (width 1) (layer "F.Cu") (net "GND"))
 (segment (start 87.89 102.14) (end 90.02 104.27) (width 0.8) (layer "F.Cu") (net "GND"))
 (segment (start 87.89 89.3) (end 87.89 102.14) (width 0.8) (layer "F.Cu") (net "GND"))
 (segment (start 95.55 72.1) (end 97.65 70) (width 0.8) (layer "F.Cu") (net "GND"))
 (segment (start 87.89 89.3) (end 87.89 87.01) (width 0.8) (layer "F.Cu") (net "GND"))
 (segment (start 126.14 72.11) (end 126.14 79.42) (width 1) (layer "F.Cu") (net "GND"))
 (segment (start 126.14 78.56) (end 126.14 79.42) (width 1) (layer "F.Cu") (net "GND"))
 (segment (start 129.62 75.08) (end 126.14 78.56) (width 1) (layer "F.Cu") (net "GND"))
 (segment (start 90.02 104.27) (end 95.4 104.27) (width 0.8) (layer "F.Cu") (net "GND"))
 (segment (start 97.65 70) (end 100 70) (width 0.8) (layer "F.Cu") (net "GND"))
 (segment (start 127.075 71.175) (end 126.14 72.11) (width 1) (layer "F.Cu") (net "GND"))
 (segment (start 128.25 70) (end 130.48 70) (width 1) (layer "F.Cu") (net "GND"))
 (segment (start 130.48 75.08) (end 133.02 75.08) (width 1) (layer "F.Cu") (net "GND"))
 (segment (start 143.7 80.2) (end 143.66 77.54) (width 1) (layer "F.Cu") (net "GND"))
 (segment (start 143.7 72.35) (end 143.7 72.4) (width 1) (layer "F.Cu") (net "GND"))
 (segment (start 143.7 77.6) (end 143.7 75.04) (width 1) (layer "F.Cu") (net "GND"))
 (via (at 122.75 67.1) (size 1.7) (drill 0.8) (layers "F.Cu" "B.Cu") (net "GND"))
 (via (at 127.075 71.175) (size 1.7) (drill 0.8) (layers "F.Cu" "B.Cu") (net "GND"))
 (segment (start 143.66 77.54) (end 143.7 77.6) (width 0.2) (layer "B.Cu") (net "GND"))
 (segment (start 126.825 71.175) (end 127.075 71.175) (width 1) (layer "B.Cu") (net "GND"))
 (segment (start 143.7 75.04) (end 143.7 75) (width 0.2) (layer "B.Cu") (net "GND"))
 (segment (start 143.7 75) (end 143.66 74.5) (width 0.2) (layer "B.Cu") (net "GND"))
 (segment (start 143.66 74.5) (end 143.7 74.46) (width 0.2) (layer "B.Cu") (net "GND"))
 (segment (start 122.75 67.1) (end 126.825 71.175) (width 1) (layer "B.Cu") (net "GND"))
 (segment (start 101.29 101.73) (end 102.54 100.48) (width 0.3) (layer "F.Cu") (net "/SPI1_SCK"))
 (segment (start 95.4 101.73) (end 101.29 101.73) (width 0.3) (layer "F.Cu") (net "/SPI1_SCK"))
 (segment (start 104.15 101.41) (end 102.54 103.02) (width 0.3) (layer "F.Cu") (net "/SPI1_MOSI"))
 (segment (start 104.15 99.65) (end 104.15 101.41) (width 0.3) (layer "F.Cu") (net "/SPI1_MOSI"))
 (segment (start 103.69 99.19) (end 104.15 99.65) (width 0.3) (layer "F.Cu") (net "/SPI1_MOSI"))
 (segment (start 95.4 99.19) (end 103.69 99.19) (width 0.3) (layer "F.Cu") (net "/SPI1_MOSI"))
 (segment (start 94.53 100.48) (end 100 100.48) (width 0.3) (layer "F.Cu") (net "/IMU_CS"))
 (segment (start 94 98.05) (end 94 99.95) (width 0.3) (layer "F.Cu") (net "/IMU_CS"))
 (segment (start 94 99.95) (end 94.53 100.48) (width 0.3) (layer "F.Cu") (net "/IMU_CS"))
 (segment (start 95.4 96.65) (end 94 98.05) (width 0.3) (layer "F.Cu") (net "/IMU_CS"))
 (segment (start 95.4 94.11) (end 93.4 96.11) (width 0.3) (layer "F.Cu") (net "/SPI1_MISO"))
 (segment (start 94.37 103.02) (end 100 103.02) (width 0.3) (layer "F.Cu") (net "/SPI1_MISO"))
 (segment (start 93.4 96.11) (end 93.4 102.05) (width 0.3) (layer "F.Cu") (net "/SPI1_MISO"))
 (segment (start 93.4 102.05) (end 94.37 103.02) (width 0.3) (layer "F.Cu") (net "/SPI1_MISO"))
 (segment (start 136 77.62) (end 133.02 77.62) (width 0.3) (layer "F.Cu") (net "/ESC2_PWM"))
 (segment (start 138.62 75) (end 136 77.62) (width 0.3) (layer "F.Cu") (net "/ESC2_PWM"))
 (segment (start 97.2 76.45) (end 98.57 75.08) (width 0.8) (layer "F.Cu") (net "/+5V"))
 (segment (start 97.2 84.25) (end 97.2 76.45) (width 0.8) (layer "F.Cu") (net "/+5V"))
 (segment (start 98.57 75.08) (end 100 75.08) (width 0.8) (layer "F.Cu") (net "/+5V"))
 (segment (start 139.9 71.65) (end 139.9 73.74) (width 0.2) (layer "F.Cu") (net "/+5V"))
 (segment (start 117.77 75.08) (end 102.54 75.08) (width 1) (layer "F.Cu") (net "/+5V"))
 (segment (start 91.15 86.8) (end 94.65 86.8) (width 0.8) (layer "F.Cu") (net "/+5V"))
 (segment (start 138.45 70.2) (end 139.9 71.65) (width 0.2) (layer "F.Cu") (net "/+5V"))
 (segment (start 139.9 73.74) (end 141.16 75) (width 0.2) (layer "F.Cu") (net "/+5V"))
 (segment (start 126.6 66.25) (end 117.77 75.08) (width 1) (layer "F.Cu") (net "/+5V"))
 (segment (start 100 75.08) (end 102.54 75.08) (width 1) (layer "F.Cu") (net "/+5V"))
 (segment (start 134.5 66.25) (end 126.6 66.25) (width 1) (layer "F.Cu") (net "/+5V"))
 (segment (start 90.43 89.3) (end 90.43 87.52) (width 0.8) (layer "F.Cu") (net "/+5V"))
 (segment (start 138.45 70.2) (end 134.5 66.25) (width 1) (layer "F.Cu") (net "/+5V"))
 (segment (start 90.43 87.52) (end 91.15 86.8) (width 0.8) (layer "F.Cu") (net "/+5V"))
 (segment (start 94.65 86.8) (end 97.2 84.25) (width 0.8) (layer "F.Cu") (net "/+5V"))
 (segment (start 137.32 78.9) (end 131.74 78.9) (width 0.3) (layer "F.Cu") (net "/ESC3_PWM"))
 (segment (start 131.74 78.9) (end 130.48 80.16) (width 0.3) (layer "F.Cu") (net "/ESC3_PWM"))
 (segment (start 138.62 77.6) (end 137.32 78.9) (width 0.3) (layer "F.Cu") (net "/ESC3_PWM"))
 (segment (start 99.157919 94.15) (end 101.29 94.15) (width 0.3) (layer "F.Cu") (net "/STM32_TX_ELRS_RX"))
 (segment (start 95.51 90.502081) (end 99.157919 94.15) (width 0.3) (layer "F.Cu") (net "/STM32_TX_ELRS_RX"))
 (segment (start 95.51 89.3) (end 95.51 90.502081) (width 0.3) (layer "F.Cu") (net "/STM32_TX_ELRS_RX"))
 (segment (start 101.29 94.15) (end 102.54 95.4) (width 0.3) (layer "F.Cu") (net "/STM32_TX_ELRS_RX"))
 (segment (start 97.5 95.95) (end 98.2 96.65) (width 0.3) (layer "F.Cu") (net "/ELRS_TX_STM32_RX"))
 (segment (start 98.2 96.65) (end 101.25 96.65) (width 0.3) (layer "F.Cu") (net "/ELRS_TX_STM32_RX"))
 (segment (start 92.97 89.32) (end 97.5 93.85) (width 0.3) (layer "F.Cu") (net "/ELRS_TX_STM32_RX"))
 (segment (start 101.25 96.65) (end 102.54 97.94) (width 0.3) (layer "F.Cu") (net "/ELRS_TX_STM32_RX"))
 (segment (start 92.97 89.3) (end 92.97 89.32) (width 0.3) (layer "F.Cu") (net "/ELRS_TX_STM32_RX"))
 (segment (start 97.5 93.85) (end 97.5 95.95) (width 0.3) (layer "F.Cu") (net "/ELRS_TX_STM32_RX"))
 (segment (start 138.62 80.2) (end 133.06 80.2) (width 0.3) (layer "F.Cu") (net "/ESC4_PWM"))
 (segment (start 133.06 80.2) (end 133.02 80.16) (width 0.3) (layer "F.Cu") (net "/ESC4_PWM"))
 (segment (start 138.62 72.4) (end 134.67 76.35) (width 0.3) (layer "F.Cu") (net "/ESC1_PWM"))
 (segment (start 131.75 76.35) (end 130.48 77.62) (width 0.3) (layer "F.Cu") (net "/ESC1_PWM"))
 (segment (start 134.67 76.35) (end 131.75 76.35) (width 0.3) (layer "F.Cu") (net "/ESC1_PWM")))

